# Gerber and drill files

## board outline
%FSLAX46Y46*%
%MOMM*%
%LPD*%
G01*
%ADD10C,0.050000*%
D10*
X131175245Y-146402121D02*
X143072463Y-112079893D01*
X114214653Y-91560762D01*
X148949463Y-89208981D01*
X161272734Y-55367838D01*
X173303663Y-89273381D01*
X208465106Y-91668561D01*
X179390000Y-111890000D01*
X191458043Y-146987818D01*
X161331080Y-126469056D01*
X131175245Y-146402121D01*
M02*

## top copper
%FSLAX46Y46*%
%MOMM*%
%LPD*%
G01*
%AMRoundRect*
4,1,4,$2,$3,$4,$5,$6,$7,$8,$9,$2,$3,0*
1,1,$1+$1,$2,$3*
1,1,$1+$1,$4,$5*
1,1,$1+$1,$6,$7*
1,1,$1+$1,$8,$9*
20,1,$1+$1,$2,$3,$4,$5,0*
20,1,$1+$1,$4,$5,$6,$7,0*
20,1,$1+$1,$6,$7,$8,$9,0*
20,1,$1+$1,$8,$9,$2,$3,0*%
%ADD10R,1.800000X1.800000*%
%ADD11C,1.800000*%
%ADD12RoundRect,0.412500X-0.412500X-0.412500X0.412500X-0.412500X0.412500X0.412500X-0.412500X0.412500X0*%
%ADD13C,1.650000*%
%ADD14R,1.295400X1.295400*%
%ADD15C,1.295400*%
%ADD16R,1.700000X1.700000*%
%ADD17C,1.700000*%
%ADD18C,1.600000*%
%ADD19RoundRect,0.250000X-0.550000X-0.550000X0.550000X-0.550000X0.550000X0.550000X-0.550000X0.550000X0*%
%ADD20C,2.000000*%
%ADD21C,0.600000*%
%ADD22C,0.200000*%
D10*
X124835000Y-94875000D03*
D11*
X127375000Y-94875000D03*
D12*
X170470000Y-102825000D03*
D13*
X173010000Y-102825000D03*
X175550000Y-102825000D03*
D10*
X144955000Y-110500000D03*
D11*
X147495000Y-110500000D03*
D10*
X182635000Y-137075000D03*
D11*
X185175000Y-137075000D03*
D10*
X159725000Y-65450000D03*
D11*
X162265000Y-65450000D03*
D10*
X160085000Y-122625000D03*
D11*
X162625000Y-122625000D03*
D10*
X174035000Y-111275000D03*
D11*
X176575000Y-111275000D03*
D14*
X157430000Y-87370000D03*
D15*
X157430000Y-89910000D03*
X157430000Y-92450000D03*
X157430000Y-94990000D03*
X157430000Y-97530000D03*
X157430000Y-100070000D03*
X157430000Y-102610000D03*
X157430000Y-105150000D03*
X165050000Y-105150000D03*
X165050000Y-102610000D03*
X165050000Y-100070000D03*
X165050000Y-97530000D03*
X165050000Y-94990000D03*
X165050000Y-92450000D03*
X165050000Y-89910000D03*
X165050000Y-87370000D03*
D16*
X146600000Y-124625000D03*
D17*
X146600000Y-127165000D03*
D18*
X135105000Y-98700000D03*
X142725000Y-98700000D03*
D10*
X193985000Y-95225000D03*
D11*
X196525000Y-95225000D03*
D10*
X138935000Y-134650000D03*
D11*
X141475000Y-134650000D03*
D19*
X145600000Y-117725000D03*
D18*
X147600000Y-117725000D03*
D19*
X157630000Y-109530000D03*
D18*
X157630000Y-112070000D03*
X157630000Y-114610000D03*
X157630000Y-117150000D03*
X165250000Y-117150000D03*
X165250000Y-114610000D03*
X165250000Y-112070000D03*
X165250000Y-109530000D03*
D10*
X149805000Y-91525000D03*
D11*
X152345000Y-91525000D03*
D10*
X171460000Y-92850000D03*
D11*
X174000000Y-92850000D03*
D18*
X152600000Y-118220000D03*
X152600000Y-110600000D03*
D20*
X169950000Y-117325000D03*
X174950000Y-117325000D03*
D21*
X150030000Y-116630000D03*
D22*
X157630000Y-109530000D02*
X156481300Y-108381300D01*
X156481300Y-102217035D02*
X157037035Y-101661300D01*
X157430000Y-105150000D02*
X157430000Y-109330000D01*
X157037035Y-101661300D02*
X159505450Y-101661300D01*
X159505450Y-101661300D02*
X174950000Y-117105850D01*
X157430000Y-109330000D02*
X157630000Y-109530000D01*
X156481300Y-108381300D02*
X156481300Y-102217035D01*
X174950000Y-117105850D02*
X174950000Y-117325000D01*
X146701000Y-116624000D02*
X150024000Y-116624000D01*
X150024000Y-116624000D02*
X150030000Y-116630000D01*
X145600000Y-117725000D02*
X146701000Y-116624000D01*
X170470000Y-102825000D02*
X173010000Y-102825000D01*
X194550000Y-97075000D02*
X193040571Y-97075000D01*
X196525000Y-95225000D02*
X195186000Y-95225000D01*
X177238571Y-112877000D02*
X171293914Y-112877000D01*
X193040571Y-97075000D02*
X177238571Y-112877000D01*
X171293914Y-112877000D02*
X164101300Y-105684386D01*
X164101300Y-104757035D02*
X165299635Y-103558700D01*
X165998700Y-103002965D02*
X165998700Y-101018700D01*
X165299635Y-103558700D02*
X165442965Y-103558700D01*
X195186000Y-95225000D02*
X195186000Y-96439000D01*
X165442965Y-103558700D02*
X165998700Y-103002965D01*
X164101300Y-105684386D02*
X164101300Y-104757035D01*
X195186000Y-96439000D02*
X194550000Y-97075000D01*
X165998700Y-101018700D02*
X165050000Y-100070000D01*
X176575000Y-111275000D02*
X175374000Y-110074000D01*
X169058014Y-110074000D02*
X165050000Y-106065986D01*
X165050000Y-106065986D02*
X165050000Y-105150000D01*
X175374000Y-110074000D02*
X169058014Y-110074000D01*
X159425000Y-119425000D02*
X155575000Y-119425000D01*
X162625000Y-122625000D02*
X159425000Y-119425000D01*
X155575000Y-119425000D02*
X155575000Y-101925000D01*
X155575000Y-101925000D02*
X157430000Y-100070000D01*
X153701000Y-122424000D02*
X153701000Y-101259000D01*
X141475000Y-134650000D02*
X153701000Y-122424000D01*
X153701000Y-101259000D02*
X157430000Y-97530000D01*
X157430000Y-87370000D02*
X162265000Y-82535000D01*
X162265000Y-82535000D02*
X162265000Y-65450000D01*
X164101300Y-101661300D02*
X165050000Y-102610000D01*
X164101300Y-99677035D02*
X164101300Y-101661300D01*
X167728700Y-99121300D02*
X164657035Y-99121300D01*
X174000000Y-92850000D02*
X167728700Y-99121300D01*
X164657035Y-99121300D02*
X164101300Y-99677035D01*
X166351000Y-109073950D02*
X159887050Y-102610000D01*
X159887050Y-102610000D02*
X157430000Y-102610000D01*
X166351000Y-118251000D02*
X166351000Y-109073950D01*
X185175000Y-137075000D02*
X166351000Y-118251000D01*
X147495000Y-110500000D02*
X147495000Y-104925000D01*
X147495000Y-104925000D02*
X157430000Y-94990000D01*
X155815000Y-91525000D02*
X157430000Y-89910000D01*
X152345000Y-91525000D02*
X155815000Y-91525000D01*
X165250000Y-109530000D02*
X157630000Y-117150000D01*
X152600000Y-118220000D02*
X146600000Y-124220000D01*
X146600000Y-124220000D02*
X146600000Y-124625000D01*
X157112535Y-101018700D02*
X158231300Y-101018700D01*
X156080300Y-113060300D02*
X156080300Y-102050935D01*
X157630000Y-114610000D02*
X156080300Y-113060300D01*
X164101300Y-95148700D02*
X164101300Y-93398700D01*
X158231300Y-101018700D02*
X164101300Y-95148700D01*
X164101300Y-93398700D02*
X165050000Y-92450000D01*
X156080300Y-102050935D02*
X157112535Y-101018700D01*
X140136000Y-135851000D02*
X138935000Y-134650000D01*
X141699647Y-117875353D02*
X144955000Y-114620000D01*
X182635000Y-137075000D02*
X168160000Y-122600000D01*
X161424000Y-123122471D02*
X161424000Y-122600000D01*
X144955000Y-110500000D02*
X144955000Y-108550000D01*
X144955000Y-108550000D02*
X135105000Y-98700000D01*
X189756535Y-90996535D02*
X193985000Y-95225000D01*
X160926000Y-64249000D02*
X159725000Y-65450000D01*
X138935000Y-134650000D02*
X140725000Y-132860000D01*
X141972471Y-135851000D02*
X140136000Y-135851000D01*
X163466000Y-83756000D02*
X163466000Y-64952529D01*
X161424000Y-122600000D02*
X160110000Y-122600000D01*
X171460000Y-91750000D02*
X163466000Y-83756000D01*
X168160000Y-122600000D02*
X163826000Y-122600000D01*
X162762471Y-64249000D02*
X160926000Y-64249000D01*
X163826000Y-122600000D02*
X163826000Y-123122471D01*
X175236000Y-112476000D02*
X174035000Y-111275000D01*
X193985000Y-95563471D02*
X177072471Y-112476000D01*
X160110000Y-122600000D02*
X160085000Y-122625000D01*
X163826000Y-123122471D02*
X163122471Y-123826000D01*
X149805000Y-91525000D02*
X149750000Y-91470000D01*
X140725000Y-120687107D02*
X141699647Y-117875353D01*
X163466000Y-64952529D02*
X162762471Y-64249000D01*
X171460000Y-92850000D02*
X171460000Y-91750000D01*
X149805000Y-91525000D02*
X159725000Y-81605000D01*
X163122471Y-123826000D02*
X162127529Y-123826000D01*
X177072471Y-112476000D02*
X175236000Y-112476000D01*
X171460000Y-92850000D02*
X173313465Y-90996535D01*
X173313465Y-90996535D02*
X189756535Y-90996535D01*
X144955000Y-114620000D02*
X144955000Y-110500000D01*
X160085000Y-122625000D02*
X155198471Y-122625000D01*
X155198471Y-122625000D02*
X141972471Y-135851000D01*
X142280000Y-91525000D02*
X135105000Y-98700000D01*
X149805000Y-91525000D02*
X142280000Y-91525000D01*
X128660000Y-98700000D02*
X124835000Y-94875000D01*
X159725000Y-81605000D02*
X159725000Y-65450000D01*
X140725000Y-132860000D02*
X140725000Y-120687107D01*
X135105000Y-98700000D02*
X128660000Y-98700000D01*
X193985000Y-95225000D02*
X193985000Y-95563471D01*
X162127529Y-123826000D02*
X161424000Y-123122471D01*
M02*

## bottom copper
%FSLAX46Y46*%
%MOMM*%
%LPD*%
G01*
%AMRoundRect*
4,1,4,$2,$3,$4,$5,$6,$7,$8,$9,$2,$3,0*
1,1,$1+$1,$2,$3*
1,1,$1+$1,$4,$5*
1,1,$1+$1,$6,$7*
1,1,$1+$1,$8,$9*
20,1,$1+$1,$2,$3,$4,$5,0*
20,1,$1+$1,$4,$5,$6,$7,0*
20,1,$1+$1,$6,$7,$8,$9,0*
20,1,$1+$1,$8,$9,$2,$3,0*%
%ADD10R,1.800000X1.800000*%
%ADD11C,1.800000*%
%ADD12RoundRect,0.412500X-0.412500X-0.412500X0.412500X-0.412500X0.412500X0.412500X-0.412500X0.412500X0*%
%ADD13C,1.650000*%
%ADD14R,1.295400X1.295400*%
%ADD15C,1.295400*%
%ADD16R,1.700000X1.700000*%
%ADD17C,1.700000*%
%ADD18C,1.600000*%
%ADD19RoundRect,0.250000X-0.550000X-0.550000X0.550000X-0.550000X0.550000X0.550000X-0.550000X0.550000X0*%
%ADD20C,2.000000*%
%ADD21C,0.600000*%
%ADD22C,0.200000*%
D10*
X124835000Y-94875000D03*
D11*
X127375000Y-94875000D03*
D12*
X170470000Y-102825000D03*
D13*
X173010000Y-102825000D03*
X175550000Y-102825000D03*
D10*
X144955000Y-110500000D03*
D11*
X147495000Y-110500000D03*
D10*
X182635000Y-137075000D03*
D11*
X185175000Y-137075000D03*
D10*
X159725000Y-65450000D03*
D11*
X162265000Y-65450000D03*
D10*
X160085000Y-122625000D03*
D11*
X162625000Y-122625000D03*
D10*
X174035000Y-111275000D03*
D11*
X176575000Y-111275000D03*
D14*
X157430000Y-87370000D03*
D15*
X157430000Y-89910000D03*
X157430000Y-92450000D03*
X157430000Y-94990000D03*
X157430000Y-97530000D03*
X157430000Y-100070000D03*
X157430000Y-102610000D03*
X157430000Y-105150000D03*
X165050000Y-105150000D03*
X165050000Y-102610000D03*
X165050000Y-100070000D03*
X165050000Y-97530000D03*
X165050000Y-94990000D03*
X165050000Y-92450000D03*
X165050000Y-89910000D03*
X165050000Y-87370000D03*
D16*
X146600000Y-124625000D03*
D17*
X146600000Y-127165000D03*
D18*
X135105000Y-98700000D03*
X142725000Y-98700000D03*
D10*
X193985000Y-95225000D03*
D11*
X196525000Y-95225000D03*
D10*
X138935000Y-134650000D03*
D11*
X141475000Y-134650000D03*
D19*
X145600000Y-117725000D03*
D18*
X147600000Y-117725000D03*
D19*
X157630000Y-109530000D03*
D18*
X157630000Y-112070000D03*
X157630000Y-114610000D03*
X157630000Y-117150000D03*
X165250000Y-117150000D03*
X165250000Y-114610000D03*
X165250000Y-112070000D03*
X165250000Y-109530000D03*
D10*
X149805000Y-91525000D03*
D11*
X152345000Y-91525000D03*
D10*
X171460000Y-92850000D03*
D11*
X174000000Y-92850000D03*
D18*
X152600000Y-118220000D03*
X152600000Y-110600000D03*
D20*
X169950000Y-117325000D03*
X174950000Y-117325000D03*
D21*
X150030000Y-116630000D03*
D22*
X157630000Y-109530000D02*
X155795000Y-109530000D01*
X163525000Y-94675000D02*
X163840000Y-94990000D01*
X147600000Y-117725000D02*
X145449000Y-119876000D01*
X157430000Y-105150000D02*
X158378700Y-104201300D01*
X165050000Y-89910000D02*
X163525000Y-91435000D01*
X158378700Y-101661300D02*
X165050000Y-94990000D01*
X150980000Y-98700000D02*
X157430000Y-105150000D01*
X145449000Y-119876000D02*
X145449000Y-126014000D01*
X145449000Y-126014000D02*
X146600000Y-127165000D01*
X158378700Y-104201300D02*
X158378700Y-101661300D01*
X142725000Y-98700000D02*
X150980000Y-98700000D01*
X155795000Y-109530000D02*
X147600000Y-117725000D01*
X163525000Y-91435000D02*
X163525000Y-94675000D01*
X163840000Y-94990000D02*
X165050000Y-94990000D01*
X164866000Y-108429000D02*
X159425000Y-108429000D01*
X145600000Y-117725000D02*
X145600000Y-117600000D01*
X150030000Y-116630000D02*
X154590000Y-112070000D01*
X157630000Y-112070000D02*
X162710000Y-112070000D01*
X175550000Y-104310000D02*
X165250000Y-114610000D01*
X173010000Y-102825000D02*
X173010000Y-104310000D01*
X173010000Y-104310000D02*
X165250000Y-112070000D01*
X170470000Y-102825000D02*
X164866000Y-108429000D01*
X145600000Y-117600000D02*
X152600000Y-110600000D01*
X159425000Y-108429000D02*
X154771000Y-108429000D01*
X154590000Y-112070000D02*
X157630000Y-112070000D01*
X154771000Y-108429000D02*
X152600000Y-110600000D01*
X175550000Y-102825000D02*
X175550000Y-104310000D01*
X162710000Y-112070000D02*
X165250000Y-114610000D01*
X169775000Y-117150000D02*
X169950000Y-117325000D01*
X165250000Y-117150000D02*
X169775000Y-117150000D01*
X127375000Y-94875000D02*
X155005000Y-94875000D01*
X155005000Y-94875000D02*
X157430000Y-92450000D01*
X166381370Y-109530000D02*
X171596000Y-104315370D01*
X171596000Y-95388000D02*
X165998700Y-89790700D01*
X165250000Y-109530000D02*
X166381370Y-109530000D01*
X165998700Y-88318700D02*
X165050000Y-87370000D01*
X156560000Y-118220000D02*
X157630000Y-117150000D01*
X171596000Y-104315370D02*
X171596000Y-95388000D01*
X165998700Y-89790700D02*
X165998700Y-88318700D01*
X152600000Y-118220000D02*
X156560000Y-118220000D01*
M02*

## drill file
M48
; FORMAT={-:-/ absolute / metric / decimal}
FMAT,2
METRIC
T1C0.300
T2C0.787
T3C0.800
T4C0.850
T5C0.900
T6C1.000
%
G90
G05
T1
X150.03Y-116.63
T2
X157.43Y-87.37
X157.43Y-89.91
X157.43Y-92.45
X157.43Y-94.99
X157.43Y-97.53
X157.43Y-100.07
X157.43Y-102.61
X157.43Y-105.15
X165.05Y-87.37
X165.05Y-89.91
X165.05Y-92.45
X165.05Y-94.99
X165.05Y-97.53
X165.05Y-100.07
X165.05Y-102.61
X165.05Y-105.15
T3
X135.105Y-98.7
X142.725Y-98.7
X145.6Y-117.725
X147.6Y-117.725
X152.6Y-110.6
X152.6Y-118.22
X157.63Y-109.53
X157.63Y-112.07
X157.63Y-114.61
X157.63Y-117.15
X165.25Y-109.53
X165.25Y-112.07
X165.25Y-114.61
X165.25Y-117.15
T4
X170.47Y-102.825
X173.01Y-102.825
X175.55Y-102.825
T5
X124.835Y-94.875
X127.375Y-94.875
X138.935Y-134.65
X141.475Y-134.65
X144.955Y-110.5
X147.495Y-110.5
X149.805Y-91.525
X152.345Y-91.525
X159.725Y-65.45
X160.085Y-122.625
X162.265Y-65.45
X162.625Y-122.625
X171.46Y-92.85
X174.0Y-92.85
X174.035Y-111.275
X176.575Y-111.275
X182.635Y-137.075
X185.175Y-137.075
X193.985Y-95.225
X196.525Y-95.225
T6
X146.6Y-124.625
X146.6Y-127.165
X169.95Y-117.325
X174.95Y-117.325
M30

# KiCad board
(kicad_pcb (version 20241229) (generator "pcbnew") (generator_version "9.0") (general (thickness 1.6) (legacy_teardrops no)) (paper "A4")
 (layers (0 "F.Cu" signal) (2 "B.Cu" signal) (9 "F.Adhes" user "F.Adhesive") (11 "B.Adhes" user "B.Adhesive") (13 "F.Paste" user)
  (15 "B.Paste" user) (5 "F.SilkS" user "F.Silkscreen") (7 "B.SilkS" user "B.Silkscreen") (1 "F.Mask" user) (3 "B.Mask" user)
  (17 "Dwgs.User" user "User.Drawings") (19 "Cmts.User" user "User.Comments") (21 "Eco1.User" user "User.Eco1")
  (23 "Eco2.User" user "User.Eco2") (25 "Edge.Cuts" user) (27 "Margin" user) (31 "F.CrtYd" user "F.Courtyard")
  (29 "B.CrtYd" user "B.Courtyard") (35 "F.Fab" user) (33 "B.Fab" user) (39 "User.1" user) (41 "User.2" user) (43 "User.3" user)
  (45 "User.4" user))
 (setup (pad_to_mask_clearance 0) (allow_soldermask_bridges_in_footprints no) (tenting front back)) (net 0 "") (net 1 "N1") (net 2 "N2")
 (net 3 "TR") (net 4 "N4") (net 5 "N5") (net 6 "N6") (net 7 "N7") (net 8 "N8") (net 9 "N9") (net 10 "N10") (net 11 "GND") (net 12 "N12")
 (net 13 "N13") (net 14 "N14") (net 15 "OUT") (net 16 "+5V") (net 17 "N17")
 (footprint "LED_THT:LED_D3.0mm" (layer "F.Cu") (at 124.835 94.875)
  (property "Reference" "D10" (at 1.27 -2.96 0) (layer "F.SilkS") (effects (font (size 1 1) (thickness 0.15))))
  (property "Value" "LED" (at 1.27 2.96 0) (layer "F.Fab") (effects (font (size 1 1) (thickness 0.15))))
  (pad "1" thru_hole rect (at 0 0) (size 1.8 1.8) (drill 0.9) (layers "*.Cu" "*.Mask") (remove_unused_layers no) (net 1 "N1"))
  (pad "2" thru_hole circle (at 2.54 0) (size 1.8 1.8) (drill 0.9) (layers "*.Cu" "*.Mask") (remove_unused_layers no) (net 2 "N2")))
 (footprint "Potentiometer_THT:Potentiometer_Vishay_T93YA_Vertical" (layer "F.Cu") (at 170.47 102.825)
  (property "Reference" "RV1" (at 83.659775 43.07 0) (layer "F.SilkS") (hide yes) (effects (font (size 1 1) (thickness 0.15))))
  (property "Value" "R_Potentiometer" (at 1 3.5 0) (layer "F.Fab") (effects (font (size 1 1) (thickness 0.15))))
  (pad "1" thru_hole roundrect (at 0 0) (size 1.65 1.65) (drill 0.85) (layers "*.Cu" "*.Mask") (remove_unused_layers no)
   (roundrect_rratio 0.25) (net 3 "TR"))
  (pad "2" thru_hole circle (at 2.54 0) (size 1.65 1.65) (drill 0.85) (layers "*.Cu" "*.Mask") (remove_unused_layers no) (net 3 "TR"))
  (pad "3" thru_hole circle (at 5.08 0) (size 1.65 1.65) (drill 0.85) (layers "*.Cu" "*.Mask") (remove_unused_layers no) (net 3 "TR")))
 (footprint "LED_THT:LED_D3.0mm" (layer "F.Cu") (at 144.955 110.5)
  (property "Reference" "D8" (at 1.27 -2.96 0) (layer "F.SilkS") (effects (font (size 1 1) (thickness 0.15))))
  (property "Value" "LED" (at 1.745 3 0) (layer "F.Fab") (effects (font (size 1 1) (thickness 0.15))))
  (pad "1" thru_hole rect (at 0 0) (size 1.8 1.8) (drill 0.9) (layers "*.Cu" "*.Mask") (remove_unused_layers no) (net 1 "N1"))
  (pad "2" thru_hole circle (at 2.54 0) (size 1.8 1.8) (drill 0.9) (layers "*.Cu" "*.Mask") (remove_unused_layers no) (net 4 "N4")))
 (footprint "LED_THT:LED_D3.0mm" (layer "F.Cu") (at 182.635 137.075)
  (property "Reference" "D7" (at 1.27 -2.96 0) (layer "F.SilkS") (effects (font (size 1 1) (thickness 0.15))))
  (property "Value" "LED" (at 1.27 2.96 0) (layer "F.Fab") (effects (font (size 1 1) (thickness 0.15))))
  (pad "1" thru_hole rect (at 0 0) (size 1.8 1.8) (drill 0.9) (layers "*.Cu" "*.Mask") (remove_unused_layers no) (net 1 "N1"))
  (pad "2" thru_hole circle (at 2.54 0) (size 1.8 1.8) (drill 0.9) (layers "*.Cu" "*.Mask") (remove_unused_layers no) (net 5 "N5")))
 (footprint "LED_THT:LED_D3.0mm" (layer "F.Cu") (at 159.725 65.45)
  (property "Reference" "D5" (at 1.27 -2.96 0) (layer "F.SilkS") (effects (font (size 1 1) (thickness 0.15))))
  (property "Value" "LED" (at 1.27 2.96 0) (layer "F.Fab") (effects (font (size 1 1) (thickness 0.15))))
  (pad "1" thru_hole rect (at 0 0) (size 1.8 1.8) (drill 0.9) (layers "*.Cu" "*.Mask") (remove_unused_layers no) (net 1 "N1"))
  (pad "2" thru_hole circle (at 2.54 0) (size 1.8 1.8) (drill 0.9) (layers "*.Cu" "*.Mask") (remove_unused_layers no) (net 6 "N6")))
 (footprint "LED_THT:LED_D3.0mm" (layer "F.Cu") (at 160.085 122.625)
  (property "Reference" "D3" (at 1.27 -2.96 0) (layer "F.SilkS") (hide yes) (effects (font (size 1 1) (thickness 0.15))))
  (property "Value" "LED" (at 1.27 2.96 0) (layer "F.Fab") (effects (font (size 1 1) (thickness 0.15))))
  (pad "1" thru_hole rect (at 0 0) (size 1.8 1.8) (drill 0.9) (layers "*.Cu" "*.Mask") (remove_unused_layers no) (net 1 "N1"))
  (pad "2" thru_hole circle (at 2.54 0) (size 1.8 1.8) (drill 0.9) (layers "*.Cu" "*.Mask") (remove_unused_layers no) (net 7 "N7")))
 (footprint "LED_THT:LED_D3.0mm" (layer "F.Cu") (at 174.035 111.275)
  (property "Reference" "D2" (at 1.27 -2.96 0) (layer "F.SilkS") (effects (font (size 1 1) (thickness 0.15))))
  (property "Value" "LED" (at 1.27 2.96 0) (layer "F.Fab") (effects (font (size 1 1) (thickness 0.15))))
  (pad "1" thru_hole rect (at 0 0) (size 1.8 1.8) (drill 0.9) (layers "*.Cu" "*.Mask") (remove_unused_layers no) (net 1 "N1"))
  (pad "2" thru_hole circle (at 2.54 0) (size 1.8 1.8) (drill 0.9) (layers "*.Cu" "*.Mask") (remove_unused_layers no) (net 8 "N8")))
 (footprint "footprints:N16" (layer "F.Cu") (at 165.05 105.15)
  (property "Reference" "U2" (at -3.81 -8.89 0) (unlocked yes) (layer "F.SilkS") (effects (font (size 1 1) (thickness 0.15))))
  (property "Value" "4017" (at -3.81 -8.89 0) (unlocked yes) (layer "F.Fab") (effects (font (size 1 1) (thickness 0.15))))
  (pad "1" thru_hole rect (at -7.62 -17.78) (size 1.2954 1.2954) (drill 0.7874) (layers "*.Cu" "*.Mask") (remove_unused_layers no)
   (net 6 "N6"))
  (pad "2" thru_hole circle (at -7.62 -15.24) (size 1.2954 1.2954) (drill 0.7874) (layers "*.Cu" "*.Mask") (remove_unused_layers no)
   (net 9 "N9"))
  (pad "3" thru_hole circle (at -7.62 -12.7) (size 1.2954 1.2954) (drill 0.7874) (layers "*.Cu" "*.Mask") (remove_unused_layers no)
   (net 2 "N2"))
  (pad "4" thru_hole circle (at -7.62 -10.16) (size 1.2954 1.2954) (drill 0.7874) (layers "*.Cu" "*.Mask") (remove_unused_layers no)
   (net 4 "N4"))
  (pad "5" thru_hole circle (at -7.62 -7.62) (size 1.2954 1.2954) (drill 0.7874) (layers "*.Cu" "*.Mask") (remove_unused_layers no)
   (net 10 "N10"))
  (pad "6" thru_hole circle (at -7.62 -5.08) (size 1.2954 1.2954) (drill 0.7874) (layers "*.Cu" "*.Mask") (remove_unused_layers no)
   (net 7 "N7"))
  (pad "7" thru_hole circle (at -7.62 -2.54) (size 1.2954 1.2954) (drill 0.7874) (layers "*.Cu" "*.Mask") (remove_unused_layers no)
   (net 5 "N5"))
  (pad "8" thru_hole circle (at -7.62 0) (size 1.2954 1.2954) (drill 0.7874) (layers "*.Cu" "*.Mask") (remove_unused_layers no)
   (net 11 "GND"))
  (pad "9" thru_hole circle (at 0 0) (size 1.2954 1.2954) (drill 0.7874) (layers "*.Cu" "*.Mask") (remove_unused_layers no) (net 8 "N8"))
  (pad "10" thru_hole circle (at 0 -2.54) (size 1.2954 1.2954) (drill 0.7874) (layers "*.Cu" "*.Mask") (remove_unused_layers no)
   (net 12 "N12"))
  (pad "11" thru_hole circle (at 0 -5.08) (size 1.2954 1.2954) (drill 0.7874) (layers "*.Cu" "*.Mask") (remove_unused_layers no)
   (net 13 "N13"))
  (pad "12" thru_hole circle (at 0 -7.62) (size 1.2954 1.2954) (drill 0.7874) (layers "*.Cu" "*.Mask") (remove_unused_layers no)
   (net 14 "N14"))
  (pad "13" thru_hole circle (at 0 -10.16) (size 1.2954 1.2954) (drill 0.7874) (layers "*.Cu" "*.Mask") (remove_unused_layers no)
   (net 11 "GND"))
  (pad "14" thru_hole circle (at 0 -12.7) (size 1.2954 1.2954) (drill 0.7874) (layers "*.Cu" "*.Mask") (remove_unused_layers no)
   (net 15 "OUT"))
  (pad "15" thru_hole circle (at 0 -15.24) (size 1.2954 1.2954) (drill 0.7874) (layers "*.Cu" "*.Mask") (remove_unused_layers no)
   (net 11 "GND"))
  (pad "16" thru_hole circle (at 0 -17.78) (size 1.2954 1.2954) (drill 0.7874) (layers "*.Cu" "*.Mask") (remove_unused_layers no)
   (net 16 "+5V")))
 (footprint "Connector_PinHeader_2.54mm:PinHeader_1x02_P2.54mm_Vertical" (layer "F.Cu") (at 146.6 124.625)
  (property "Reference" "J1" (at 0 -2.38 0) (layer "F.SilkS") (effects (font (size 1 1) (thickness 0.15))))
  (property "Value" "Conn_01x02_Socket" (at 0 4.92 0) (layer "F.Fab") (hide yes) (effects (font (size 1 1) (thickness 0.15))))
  (pad "1" thru_hole rect (at 0 0) (size 1.7 1.7) (drill 1) (layers "*.Cu" "*.Mask") (remove_unused_layers no) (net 16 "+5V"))
  (pad "2" thru_hole circle (at 0 2.54) (size 1.7 1.7) (drill 1) (layers "*.Cu" "*.Mask") (remove_unused_layers no) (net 11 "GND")))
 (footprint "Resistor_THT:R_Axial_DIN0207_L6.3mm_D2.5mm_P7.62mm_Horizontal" (layer "F.Cu") (at 135.105 98.7)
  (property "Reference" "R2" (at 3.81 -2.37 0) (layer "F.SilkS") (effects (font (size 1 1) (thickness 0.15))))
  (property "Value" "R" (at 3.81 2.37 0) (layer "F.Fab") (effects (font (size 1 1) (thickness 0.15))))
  (pad "1" thru_hole circle (at 0 0) (size 1.6 1.6) (drill 0.8) (layers "*.Cu" "*.Mask") (remove_unused_layers no) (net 1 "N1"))
  (pad "2" thru_hole circle (at 7.62 0) (size 1.6 1.6) (drill 0.8) (layers "*.Cu" "*.Mask") (remove_unused_layers no) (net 11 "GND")))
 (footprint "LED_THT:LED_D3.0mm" (layer "F.Cu") (at 193.985 95.225)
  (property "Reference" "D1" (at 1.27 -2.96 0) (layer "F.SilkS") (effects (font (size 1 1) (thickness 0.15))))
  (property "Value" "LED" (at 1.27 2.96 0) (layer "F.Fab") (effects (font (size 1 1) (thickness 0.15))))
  (pad "1" thru_hole rect (at 0 0) (size 1.8 1.8) (drill 0.9) (layers "*.Cu" "*.Mask") (remove_unused_layers no) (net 1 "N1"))
  (pad "2" thru_hole circle (at 2.54 0) (size 1.8 1.8) (drill 0.9) (layers "*.Cu" "*.Mask") (remove_unused_layers no) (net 13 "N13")))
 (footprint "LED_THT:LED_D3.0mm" (layer "F.Cu") (at 138.935 134.65)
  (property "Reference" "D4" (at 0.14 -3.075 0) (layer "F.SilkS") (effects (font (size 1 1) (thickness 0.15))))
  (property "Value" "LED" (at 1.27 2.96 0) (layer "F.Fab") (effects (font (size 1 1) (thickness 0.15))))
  (pad "1" thru_hole rect (at 0 0) (size 1.8 1.8) (drill 0.9) (layers "*.Cu" "*.Mask") (remove_unused_layers no) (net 1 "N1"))
  (pad "2" thru_hole circle (at 2.54 0) (size 1.8 1.8) (drill 0.9) (layers "*.Cu" "*.Mask") (remove_unused_layers no) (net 10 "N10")))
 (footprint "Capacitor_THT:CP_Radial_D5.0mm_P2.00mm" (layer "F.Cu") (at 145.6 117.725)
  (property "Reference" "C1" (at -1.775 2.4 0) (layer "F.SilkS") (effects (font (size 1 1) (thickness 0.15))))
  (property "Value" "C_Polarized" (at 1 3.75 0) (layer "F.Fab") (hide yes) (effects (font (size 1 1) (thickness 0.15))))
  (pad "1" thru_hole roundrect (at 0 0) (size 1.6 1.6) (drill 0.8) (layers "*.Cu" "*.Mask") (remove_unused_layers no)
   (roundrect_rratio 0.15625) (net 3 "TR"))
  (pad "2" thru_hole circle (at 2 0) (size 1.6 1.6) (drill 0.8) (layers "*.Cu" "*.Mask") (remove_unused_layers no) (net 11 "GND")))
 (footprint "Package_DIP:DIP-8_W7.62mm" (layer "F.Cu") (at 157.63 109.53)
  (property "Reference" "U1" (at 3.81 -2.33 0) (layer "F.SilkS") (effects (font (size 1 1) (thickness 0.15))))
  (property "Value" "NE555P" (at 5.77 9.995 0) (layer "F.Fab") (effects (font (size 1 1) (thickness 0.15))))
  (pad "1" thru_hole roundrect (at 0 0) (size 1.6 1.6) (drill 0.8) (layers "*.Cu" "*.Mask") (remove_unused_layers no)
   (roundrect_rratio 0.15625) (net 11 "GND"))
  (pad "2" thru_hole circle (at 0 2.54) (size 1.6 1.6) (drill 0.8) (layers "*.Cu" "*.Mask") (remove_unused_layers no) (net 3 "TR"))
  (pad "3" thru_hole circle (at 0 5.08) (size 1.6 1.6) (drill 0.8) (layers "*.Cu" "*.Mask") (remove_unused_layers no) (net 15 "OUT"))
  (pad "4" thru_hole circle (at 0 7.62) (size 1.6 1.6) (drill 0.8) (layers "*.Cu" "*.Mask") (remove_unused_layers no) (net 16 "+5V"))
  (pad "5" thru_hole circle (at 7.62 7.62) (size 1.6 1.6) (drill 0.8) (layers "*.Cu" "*.Mask") (remove_unused_layers no) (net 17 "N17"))
  (pad "6" thru_hole circle (at 7.62 5.08) (size 1.6 1.6) (drill 0.8) (layers "*.Cu" "*.Mask") (remove_unused_layers no) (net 3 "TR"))
  (pad "7" thru_hole circle (at 7.62 2.54) (size 1.6 1.6) (drill 0.8) (layers "*.Cu" "*.Mask") (remove_unused_layers no) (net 3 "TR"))
  (pad "8" thru_hole circle (at 7.62 0) (size 1.6 1.6) (drill 0.8) (layers "*.Cu" "*.Mask") (remove_unused_layers no) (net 16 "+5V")))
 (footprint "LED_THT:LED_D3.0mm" (layer "F.Cu") (at 149.805 91.525)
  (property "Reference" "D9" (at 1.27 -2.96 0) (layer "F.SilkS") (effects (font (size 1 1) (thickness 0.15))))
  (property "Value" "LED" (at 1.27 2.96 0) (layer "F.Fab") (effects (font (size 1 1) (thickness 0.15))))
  (pad "1" thru_hole rect (at 0 0) (size 1.8 1.8) (drill 0.9) (layers "*.Cu" "*.Mask") (remove_unused_layers no) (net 1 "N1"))
  (pad "2" thru_hole circle (at 2.54 0) (size 1.8 1.8) (drill 0.9) (layers "*.Cu" "*.Mask") (remove_unused_layers no) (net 9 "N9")))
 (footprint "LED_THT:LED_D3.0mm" (layer "F.Cu") (at 171.46 92.85)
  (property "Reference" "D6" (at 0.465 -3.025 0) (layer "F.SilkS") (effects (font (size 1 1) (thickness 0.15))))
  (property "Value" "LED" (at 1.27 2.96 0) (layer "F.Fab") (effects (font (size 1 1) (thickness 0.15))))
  (pad "1" thru_hole rect (at 0 0) (size 1.8 1.8) (drill 0.9) (layers "*.Cu" "*.Mask") (remove_unused_layers no) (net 1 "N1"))
  (pad "2" thru_hole circle (at 2.54 0) (size 1.8 1.8) (drill 0.9) (layers "*.Cu" "*.Mask") (remove_unused_layers no) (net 12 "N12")))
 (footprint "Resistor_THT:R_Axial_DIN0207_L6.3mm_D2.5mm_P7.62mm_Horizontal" (layer "F.Cu") (at 152.6 118.22 90)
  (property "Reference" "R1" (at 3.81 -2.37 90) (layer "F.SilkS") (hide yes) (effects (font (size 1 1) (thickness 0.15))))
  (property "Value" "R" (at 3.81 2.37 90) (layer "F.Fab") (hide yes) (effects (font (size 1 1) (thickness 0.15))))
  (pad "1" thru_hole circle (at 0 0 90) (size 1.6 1.6) (drill 0.8) (layers "*.Cu" "*.Mask") (remove_unused_layers no) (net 16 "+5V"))
  (pad "2" thru_hole circle (at 7.62 0 90) (size 1.6 1.6) (drill 0.8) (layers "*.Cu" "*.Mask") (remove_unused_layers no) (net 3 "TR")))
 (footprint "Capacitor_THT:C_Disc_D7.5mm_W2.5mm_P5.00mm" (layer "F.Cu") (at 169.95 117.325)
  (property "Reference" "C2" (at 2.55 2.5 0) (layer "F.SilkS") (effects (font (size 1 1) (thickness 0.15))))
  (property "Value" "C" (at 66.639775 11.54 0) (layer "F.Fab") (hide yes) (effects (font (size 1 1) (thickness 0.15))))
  (pad "1" thru_hole circle (at 0 0) (size 2 2) (drill 1) (layers "*.Cu" "*.Mask") (remove_unused_layers no) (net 17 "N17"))
  (pad "2" thru_hole circle (at 5 0) (size 2 2) (drill 1) (layers "*.Cu" "*.Mask") (remove_unused_layers no) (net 11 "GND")))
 (gr_poly
  (pts (xy 131.175245 146.402121) (xy 143.072463 112.079893) (xy 114.214653 91.560762) (xy 148.949463 89.208981) (xy 161.272734 55.367838)
   (xy 173.303663 89.273381) (xy 208.465106 91.668561) (xy 179.39 111.89) (xy 191.458043 146.987818) (xy 161.33108 126.469056))
  (stroke (width 0.05) (type solid)) (fill no) (layer "Edge.Cuts"))
 (segment (start 157.63 109.53) (end 156.4813 108.3813) (width 0.2) (layer "F.Cu") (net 11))
 (segment (start 156.4813 102.217035) (end 157.037035 101.6613) (width 0.2) (layer "F.Cu") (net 11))
 (segment (start 157.43 105.15) (end 157.43 109.33) (width 0.2) (layer "F.Cu") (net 11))
 (segment (start 157.037035 101.6613) (end 159.50545 101.6613) (width 0.2) (layer "F.Cu") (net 11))
 (segment (start 159.50545 101.6613) (end 174.95 117.10585) (width 0.2) (layer "F.Cu") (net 11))
 (segment (start 157.43 109.33) (end 157.63 109.53) (width 0.2) (layer "F.Cu") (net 11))
 (segment (start 156.4813 108.3813) (end 156.4813 102.217035) (width 0.2) (layer "F.Cu") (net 11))
 (segment (start 174.95 117.10585) (end 174.95 117.325) (width 0.2) (layer "F.Cu") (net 11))
 (segment (start 157.63 109.53) (end 155.795 109.53) (width 0.2) (layer "B.Cu") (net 11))
 (segment (start 163.525 94.675) (end 163.84 94.99) (width 0.2) (layer "B.Cu") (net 11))
 (segment (start 147.6 117.725) (end 145.449 119.876) (width 0.2) (layer "B.Cu") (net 11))
 (segment (start 157.43 105.15) (end 158.3787 104.2013) (width 0.2) (layer "B.Cu") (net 11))
 (segment (start 165.05 89.91) (end 163.525 91.435) (width 0.2) (layer "B.Cu") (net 11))
 (segment (start 158.3787 101.6613) (end 165.05 94.99) (width 0.2) (layer "B.Cu") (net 11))
 (segment (start 150.98 98.7) (end 157.43 105.15) (width 0.2) (layer "B.Cu") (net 11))
 (segment (start 145.449 119.876) (end 145.449 126.014) (width 0.2) (layer "B.Cu") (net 11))
 (segment (start 145.449 126.014) (end 146.6 127.165) (width 0.2) (layer "B.Cu") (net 11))
 (segment (start 158.3787 104.2013) (end 158.3787 101.6613) (width 0.2) (layer "B.Cu") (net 11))
 (segment (start 142.725 98.7) (end 150.98 98.7) (width 0.2) (layer "B.Cu") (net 11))
 (segment (start 155.795 109.53) (end 147.6 117.725) (width 0.2) (layer "B.Cu") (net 11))
 (segment (start 163.525 91.435) (end 163.525 94.675) (width 0.2) (layer "B.Cu") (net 11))
 (segment (start 163.84 94.99) (end 165.05 94.99) (width 0.2) (layer "B.Cu") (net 11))
 (segment (start 146.701 116.624) (end 150.024 116.624) (width 0.2) (layer "F.Cu") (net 3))
 (segment (start 150.024 116.624) (end 150.03 116.63) (width 0.2) (layer "F.Cu") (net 3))
 (segment (start 145.6 117.725) (end 146.701 116.624) (width 0.2) (layer "F.Cu") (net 3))
 (segment (start 170.47 102.825) (end 173.01 102.825) (width 0.2) (layer "F.Cu") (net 3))
 (via (at 150.03 116.63) (size 0.6) (drill 0.3) (layers "F.Cu" "B.Cu") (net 3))
 (segment (start 164.866 108.429) (end 159.425 108.429) (width 0.2) (layer "B.Cu") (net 3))
 (segment (start 145.6 117.725) (end 145.6 117.6) (width 0.2) (layer "B.Cu") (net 3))
 (segment (start 150.03 116.63) (end 154.59 112.07) (width 0.2) (layer "B.Cu") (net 3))
 (segment (start 157.63 112.07) (end 162.71 112.07) (width 0.2) (layer "B.Cu") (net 3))
 (segment (start 175.55 104.31) (end 165.25 114.61) (width 0.2) (layer "B.Cu") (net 3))
 (segment (start 173.01 102.825) (end 173.01 104.31) (width 0.2) (layer "B.Cu") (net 3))
 (segment (start 173.01 104.31) (end 165.25 112.07) (width 0.2) (layer "B.Cu") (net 3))
 (segment (start 170.47 102.825) (end 164.866 108.429) (width 0.2) (layer "B.Cu") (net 3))
 (segment (start 145.6 117.6) (end 152.6 110.6) (width 0.2) (layer "B.Cu") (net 3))
 (segment (start 159.425 108.429) (end 154.771 108.429) (width 0.2) (layer "B.Cu") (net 3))
 (segment (start 154.59 112.07) (end 157.63 112.07) (width 0.2) (layer "B.Cu") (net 3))
 (segment (start 154.771 108.429) (end 152.6 110.6) (width 0.2) (layer "B.Cu") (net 3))
 (segment (start 175.55 102.825) (end 175.55 104.31) (width 0.2) (layer "B.Cu") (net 3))
 (segment (start 162.71 112.07) (end 165.25 114.61) (width 0.2) (layer "B.Cu") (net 3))
 (segment (start 169.775 117.15) (end 169.95 117.325) (width 0.2) (layer "B.Cu") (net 17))
 (segment (start 165.25 117.15) (end 169.775 117.15) (width 0.2) (layer "B.Cu") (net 17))
 (segment (start 194.55 97.075) (end 193.040571 97.075) (width 0.2) (layer "F.Cu") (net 13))
 (segment (start 196.525 95.225) (end 195.186 95.225) (width 0.2) (layer "F.Cu") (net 13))
 (segment (start 177.238571 112.877) (end 171.293914 112.877) (width 0.2) (layer "F.Cu") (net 13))
 (segment (start 193.040571 97.075) (end 177.238571 112.877) (width 0.2) (layer "F.Cu") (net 13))
 (segment (start 171.293914 112.877) (end 164.1013 105.684386) (width 0.2) (layer "F.Cu") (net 13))
 (segment (start 164.1013 104.757035) (end 165.299635 103.5587) (width 0.2) (layer "F.Cu") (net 13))
 (segment (start 165.9987 103.002965) (end 165.9987 101.0187) (width 0.2) (layer "F.Cu") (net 13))
 (segment (start 165.299635 103.5587) (end 165.442965 103.5587) (width 0.2) (layer "F.Cu") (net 13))
 (segment (start 195.186 95.225) (end 195.186 96.439) (width 0.2) (layer "F.Cu") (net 13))
 (segment (start 165.442965 103.5587) (end 165.9987 103.002965) (width 0.2) (layer "F.Cu") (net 13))
 (segment (start 164.1013 105.684386) (end 164.1013 104.757035) (width 0.2) (layer "F.Cu") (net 13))
 (segment (start 195.186 96.439) (end 194.55 97.075) (width 0.2) (layer "F.Cu") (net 13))
 (segment (start 165.9987 101.0187) (end 165.05 100.07) (width 0.2) (layer "F.Cu") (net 13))
 (segment (start 176.575 111.275) (end 175.374 110.074) (width 0.2) (layer "F.Cu") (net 8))
 (segment (start 169.058014 110.074) (end 165.05 106.065986) (width 0.2) (layer "F.Cu") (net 8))
 (segment (start 165.05 106.065986) (end 165.05 105.15) (width 0.2) (layer "F.Cu") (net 8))
 (segment (start 175.374 110.074) (end 169.058014 110.074) (width 0.2) (layer "F.Cu") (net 8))
 (segment (start 159.425 119.425) (end 155.575 119.425) (width 0.2) (layer "F.Cu") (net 7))
 (segment (start 162.625 122.625) (end 159.425 119.425) (width 0.2) (layer "F.Cu") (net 7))
 (segment (start 155.575 119.425) (end 155.575 101.925) (width 0.2) (layer "F.Cu") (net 7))
 (segment (start 155.575 101.925) (end 157.43 100.07) (width 0.2) (layer "F.Cu") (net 7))
 (segment (start 153.701 122.424) (end 153.701 101.259) (width 0.2) (layer "F.Cu") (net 10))
 (segment (start 141.475 134.65) (end 153.701 122.424) (width 0.2) (layer "F.Cu") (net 10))
 (segment (start 153.701 101.259) (end 157.43 97.53) (width 0.2) (layer "F.Cu") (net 10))
 (segment (start 157.43 87.37) (end 162.265 82.535) (width 0.2) (layer "F.Cu") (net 6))
 (segment (start 162.265 82.535) (end 162.265 65.45) (width 0.2) (layer "F.Cu") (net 6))
 (segment (start 164.1013 101.6613) (end 165.05 102.61) (width 0.2) (layer "F.Cu") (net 12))
 (segment (start 164.1013 99.677035) (end 164.1013 101.6613) (width 0.2) (layer "F.Cu") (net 12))
 (segment (start 167.7287 99.1213) (end 164.657035 99.1213) (width 0.2) (layer "F.Cu") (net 12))
 (segment (start 174 92.85) (end 167.7287 99.1213) (width 0.2) (layer "F.Cu") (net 12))
 (segment (start 164.657035 99.1213) (end 164.1013 99.677035) (width 0.2) (layer "F.Cu") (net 12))
 (segment (start 166.351 109.07395) (end 159.88705 102.61) (width 0.2) (layer "F.Cu") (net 5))
 (segment (start 159.88705 102.61) (end 157.43 102.61) (width 0.2) (layer "F.Cu") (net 5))
 (segment (start 166.351 118.251) (end 166.351 109.07395) (width 0.2) (layer "F.Cu") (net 5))
 (segment (start 185.175 137.075) (end 166.351 118.251) (width 0.2) (layer "F.Cu") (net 5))
 (segment (start 147.495 110.5) (end 147.495 104.925) (width 0.2) (layer "F.Cu") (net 4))
 (segment (start 147.495 104.925) (end 157.43 94.99) (width 0.2) (layer "F.Cu") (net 4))
 (segment (start 155.815 91.525) (end 157.43 89.91) (width 0.2) (layer "F.Cu") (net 9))
 (segment (start 152.345 91.525) (end 155.815 91.525) (width 0.2) (layer "F.Cu") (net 9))
 (segment (start 127.375 94.875) (end 155.005 94.875) (width 0.2) (layer "B.Cu") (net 2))
 (segment (start 155.005 94.875) (end 157.43 92.45) (width 0.2) (layer "B.Cu") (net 2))
 (segment (start 165.25 109.53) (end 157.63 117.15) (width 0.2) (layer "F.Cu") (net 16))
 (segment (start 152.6 118.22) (end 146.6 124.22) (width 0.2) (layer "F.Cu") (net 16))
 (segment (start 146.6 124.22) (end 146.6 124.625) (width 0.2) (layer "F.Cu") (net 16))
 (segment (start 166.38137 109.53) (end 171.596 104.31537) (width 0.2) (layer "B.Cu") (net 16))
 (segment (start 171.596 95.388) (end 165.9987 89.7907) (width 0.2) (layer "B.Cu") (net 16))
 (segment (start 165.25 109.53) (end 166.38137 109.53) (width 0.2) (layer "B.Cu") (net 16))
 (segment (start 165.9987 88.3187) (end 165.05 87.37) (width 0.2) (layer "B.Cu") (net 16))
 (segment (start 156.56 118.22) (end 157.63 117.15) (width 0.2) (layer "B.Cu") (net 16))
 (segment (start 171.596 104.31537) (end 171.596 95.388) (width 0.2) (layer "B.Cu") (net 16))
 (segment (start 165.9987 89.7907) (end 165.9987 88.3187) (width 0.2) (layer "B.Cu") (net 16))
 (segment (start 152.6 118.22) (end 156.56 118.22) (width 0.2) (layer "B.Cu") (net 16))
 (segment (start 157.112535 101.0187) (end 158.2313 101.0187) (width 0.2) (layer "F.Cu") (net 15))
 (segment (start 156.0803 113.0603) (end 156.0803 102.050935) (width 0.2) (layer "F.Cu") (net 15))
 (segment (start 157.63 114.61) (end 156.0803 113.0603) (width 0.2) (layer "F.Cu") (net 15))
 (segment (start 164.1013 95.1487) (end 164.1013 93.3987) (width 0.2) (layer "F.Cu") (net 15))
 (segment (start 158.2313 101.0187) (end 164.1013 95.1487) (width 0.2) (layer "F.Cu") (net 15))
 (segment (start 164.1013 93.3987) (end 165.05 92.45) (width 0.2) (layer "F.Cu") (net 15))
 (segment (start 156.0803 102.050935) (end 157.112535 101.0187) (width 0.2) (layer "F.Cu") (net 15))
 (segment (start 140.136 135.851) (end 138.935 134.65) (width 0.2) (layer "F.Cu") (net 1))
 (segment (start 141.699647 117.875353) (end 144.955 114.62) (width 0.2) (layer "F.Cu") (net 1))
 (segment (start 182.635 137.075) (end 168.16 122.6) (width 0.2) (layer "F.Cu") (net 1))
 (segment (start 161.424 123.122471) (end 161.424 122.6) (width 0.2) (layer "F.Cu") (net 1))
 (segment (start 144.955 110.5) (end 144.955 108.55) (width 0.2) (layer "F.Cu") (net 1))
 (segment (start 144.955 108.55) (end 135.105 98.7) (width 0.2) (layer "F.Cu") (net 1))
 (segment (start 189.756535 90.996535) (end 193.985 95.225) (width 0.2) (layer "F.Cu") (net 1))
 (segment (start 160.926 64.249) (end 159.725 65.45) (width 0.2) (layer "F.Cu") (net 1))
 (segment (start 138.935 134.65) (end 140.725 132.86) (width 0.2) (layer "F.Cu") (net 1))
 (segment (start 141.972471 135.851) (end 140.136 135.851) (width 0.2) (layer "F.Cu") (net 1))
 (segment (start 163.466 83.756) (end 163.466 64.952529) (width 0.2) (layer "F.Cu") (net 1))
 (segment (start 161.424 122.6) (end 160.11 122.6) (width 0.2) (layer "F.Cu") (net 1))
 (segment (start 171.46 91.75) (end 163.466 83.756) (width 0.2) (layer "F.Cu") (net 1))
 (segment (start 168.16 122.6) (end 163.826 122.6) (width 0.2) (layer "F.Cu") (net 1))
 (segment (start 162.762471 64.249) (end 160.926 64.249) (width 0.2) (layer "F.Cu") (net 1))
 (segment (start 163.826 122.6) (end 163.826 123.122471) (width 0.2) (layer "F.Cu") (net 1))
 (segment (start 175.236 112.476) (end 174.035 111.275) (width 0.2) (layer "F.Cu") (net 1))
 (segment (start 193.985 95.563471) (end 177.072471 112.476) (width 0.2) (layer "F.Cu") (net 1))
 (segment (start 160.11 122.6) (end 160.085 122.625) (width 0.2) (layer "F.Cu") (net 1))
 (segment (start 163.826 123.122471) (end 163.122471 123.826) (width 0.2) (layer "F.Cu") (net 1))
 (segment (start 149.805 91.525) (end 149.75 91.47) (width 0.2) (layer "F.Cu") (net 1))
 (segment (start 140.725 120.687107) (end 141.699647 117.875353) (width 0.2) (layer "F.Cu") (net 1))
 (segment (start 163.466 64.952529) (end 162.762471 64.249) (width 0.2) (layer "F.Cu") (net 1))
 (segment (start 171.46 92.85) (end 171.46 91.75) (width 0.2) (layer "F.Cu") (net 1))
 (segment (start 149.805 91.525) (end 159.725 81.605) (width 0.2) (layer "F.Cu") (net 1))
 (segment (start 163.122471 123.826) (end 162.127529 123.826) (width 0.2) (layer "F.Cu") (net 1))
 (segment (start 177.072471 112.476) (end 175.236 112.476) (width 0.2) (layer "F.Cu") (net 1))
 (segment (start 171.46 92.85) (end 173.313465 90.996535) (width 0.2) (layer "F.Cu") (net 1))
 (segment (start 173.313465 90.996535) (end 189.756535 90.996535) (width 0.2) (layer "F.Cu") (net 1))
 (segment (start 144.955 114.62) (end 144.955 110.5) (width 0.2) (layer "F.Cu") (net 1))
 (segment (start 160.085 122.625) (end 155.198471 122.625) (width 0.2) (layer "F.Cu") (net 1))
 (segment (start 155.198471 122.625) (end 141.972471 135.851) (width 0.2) (layer "F.Cu") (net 1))
 (segment (start 142.28 91.525) (end 135.105 98.7) (width 0.2) (layer "F.Cu") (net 1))
 (segment (start 149.805 91.525) (end 142.28 91.525) (width 0.2) (layer "F.Cu") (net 1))
 (segment (start 128.66 98.7) (end 124.835 94.875) (width 0.2) (layer "F.Cu") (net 1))
 (segment (start 159.725 81.605) (end 159.725 65.45) (width 0.2) (layer "F.Cu") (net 1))
 (segment (start 140.725 132.86) (end 140.725 120.687107) (width 0.2) (layer "F.Cu") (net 1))
 (segment (start 135.105 98.7) (end 128.66 98.7) (width 0.2) (layer "F.Cu") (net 1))
 (segment (start 193.985 95.225) (end 193.985 95.563471) (width 0.2) (layer "F.Cu") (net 1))
 (segment (start 162.127529 123.826) (end 161.424 123.122471) (width 0.2) (layer "F.Cu") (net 1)))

